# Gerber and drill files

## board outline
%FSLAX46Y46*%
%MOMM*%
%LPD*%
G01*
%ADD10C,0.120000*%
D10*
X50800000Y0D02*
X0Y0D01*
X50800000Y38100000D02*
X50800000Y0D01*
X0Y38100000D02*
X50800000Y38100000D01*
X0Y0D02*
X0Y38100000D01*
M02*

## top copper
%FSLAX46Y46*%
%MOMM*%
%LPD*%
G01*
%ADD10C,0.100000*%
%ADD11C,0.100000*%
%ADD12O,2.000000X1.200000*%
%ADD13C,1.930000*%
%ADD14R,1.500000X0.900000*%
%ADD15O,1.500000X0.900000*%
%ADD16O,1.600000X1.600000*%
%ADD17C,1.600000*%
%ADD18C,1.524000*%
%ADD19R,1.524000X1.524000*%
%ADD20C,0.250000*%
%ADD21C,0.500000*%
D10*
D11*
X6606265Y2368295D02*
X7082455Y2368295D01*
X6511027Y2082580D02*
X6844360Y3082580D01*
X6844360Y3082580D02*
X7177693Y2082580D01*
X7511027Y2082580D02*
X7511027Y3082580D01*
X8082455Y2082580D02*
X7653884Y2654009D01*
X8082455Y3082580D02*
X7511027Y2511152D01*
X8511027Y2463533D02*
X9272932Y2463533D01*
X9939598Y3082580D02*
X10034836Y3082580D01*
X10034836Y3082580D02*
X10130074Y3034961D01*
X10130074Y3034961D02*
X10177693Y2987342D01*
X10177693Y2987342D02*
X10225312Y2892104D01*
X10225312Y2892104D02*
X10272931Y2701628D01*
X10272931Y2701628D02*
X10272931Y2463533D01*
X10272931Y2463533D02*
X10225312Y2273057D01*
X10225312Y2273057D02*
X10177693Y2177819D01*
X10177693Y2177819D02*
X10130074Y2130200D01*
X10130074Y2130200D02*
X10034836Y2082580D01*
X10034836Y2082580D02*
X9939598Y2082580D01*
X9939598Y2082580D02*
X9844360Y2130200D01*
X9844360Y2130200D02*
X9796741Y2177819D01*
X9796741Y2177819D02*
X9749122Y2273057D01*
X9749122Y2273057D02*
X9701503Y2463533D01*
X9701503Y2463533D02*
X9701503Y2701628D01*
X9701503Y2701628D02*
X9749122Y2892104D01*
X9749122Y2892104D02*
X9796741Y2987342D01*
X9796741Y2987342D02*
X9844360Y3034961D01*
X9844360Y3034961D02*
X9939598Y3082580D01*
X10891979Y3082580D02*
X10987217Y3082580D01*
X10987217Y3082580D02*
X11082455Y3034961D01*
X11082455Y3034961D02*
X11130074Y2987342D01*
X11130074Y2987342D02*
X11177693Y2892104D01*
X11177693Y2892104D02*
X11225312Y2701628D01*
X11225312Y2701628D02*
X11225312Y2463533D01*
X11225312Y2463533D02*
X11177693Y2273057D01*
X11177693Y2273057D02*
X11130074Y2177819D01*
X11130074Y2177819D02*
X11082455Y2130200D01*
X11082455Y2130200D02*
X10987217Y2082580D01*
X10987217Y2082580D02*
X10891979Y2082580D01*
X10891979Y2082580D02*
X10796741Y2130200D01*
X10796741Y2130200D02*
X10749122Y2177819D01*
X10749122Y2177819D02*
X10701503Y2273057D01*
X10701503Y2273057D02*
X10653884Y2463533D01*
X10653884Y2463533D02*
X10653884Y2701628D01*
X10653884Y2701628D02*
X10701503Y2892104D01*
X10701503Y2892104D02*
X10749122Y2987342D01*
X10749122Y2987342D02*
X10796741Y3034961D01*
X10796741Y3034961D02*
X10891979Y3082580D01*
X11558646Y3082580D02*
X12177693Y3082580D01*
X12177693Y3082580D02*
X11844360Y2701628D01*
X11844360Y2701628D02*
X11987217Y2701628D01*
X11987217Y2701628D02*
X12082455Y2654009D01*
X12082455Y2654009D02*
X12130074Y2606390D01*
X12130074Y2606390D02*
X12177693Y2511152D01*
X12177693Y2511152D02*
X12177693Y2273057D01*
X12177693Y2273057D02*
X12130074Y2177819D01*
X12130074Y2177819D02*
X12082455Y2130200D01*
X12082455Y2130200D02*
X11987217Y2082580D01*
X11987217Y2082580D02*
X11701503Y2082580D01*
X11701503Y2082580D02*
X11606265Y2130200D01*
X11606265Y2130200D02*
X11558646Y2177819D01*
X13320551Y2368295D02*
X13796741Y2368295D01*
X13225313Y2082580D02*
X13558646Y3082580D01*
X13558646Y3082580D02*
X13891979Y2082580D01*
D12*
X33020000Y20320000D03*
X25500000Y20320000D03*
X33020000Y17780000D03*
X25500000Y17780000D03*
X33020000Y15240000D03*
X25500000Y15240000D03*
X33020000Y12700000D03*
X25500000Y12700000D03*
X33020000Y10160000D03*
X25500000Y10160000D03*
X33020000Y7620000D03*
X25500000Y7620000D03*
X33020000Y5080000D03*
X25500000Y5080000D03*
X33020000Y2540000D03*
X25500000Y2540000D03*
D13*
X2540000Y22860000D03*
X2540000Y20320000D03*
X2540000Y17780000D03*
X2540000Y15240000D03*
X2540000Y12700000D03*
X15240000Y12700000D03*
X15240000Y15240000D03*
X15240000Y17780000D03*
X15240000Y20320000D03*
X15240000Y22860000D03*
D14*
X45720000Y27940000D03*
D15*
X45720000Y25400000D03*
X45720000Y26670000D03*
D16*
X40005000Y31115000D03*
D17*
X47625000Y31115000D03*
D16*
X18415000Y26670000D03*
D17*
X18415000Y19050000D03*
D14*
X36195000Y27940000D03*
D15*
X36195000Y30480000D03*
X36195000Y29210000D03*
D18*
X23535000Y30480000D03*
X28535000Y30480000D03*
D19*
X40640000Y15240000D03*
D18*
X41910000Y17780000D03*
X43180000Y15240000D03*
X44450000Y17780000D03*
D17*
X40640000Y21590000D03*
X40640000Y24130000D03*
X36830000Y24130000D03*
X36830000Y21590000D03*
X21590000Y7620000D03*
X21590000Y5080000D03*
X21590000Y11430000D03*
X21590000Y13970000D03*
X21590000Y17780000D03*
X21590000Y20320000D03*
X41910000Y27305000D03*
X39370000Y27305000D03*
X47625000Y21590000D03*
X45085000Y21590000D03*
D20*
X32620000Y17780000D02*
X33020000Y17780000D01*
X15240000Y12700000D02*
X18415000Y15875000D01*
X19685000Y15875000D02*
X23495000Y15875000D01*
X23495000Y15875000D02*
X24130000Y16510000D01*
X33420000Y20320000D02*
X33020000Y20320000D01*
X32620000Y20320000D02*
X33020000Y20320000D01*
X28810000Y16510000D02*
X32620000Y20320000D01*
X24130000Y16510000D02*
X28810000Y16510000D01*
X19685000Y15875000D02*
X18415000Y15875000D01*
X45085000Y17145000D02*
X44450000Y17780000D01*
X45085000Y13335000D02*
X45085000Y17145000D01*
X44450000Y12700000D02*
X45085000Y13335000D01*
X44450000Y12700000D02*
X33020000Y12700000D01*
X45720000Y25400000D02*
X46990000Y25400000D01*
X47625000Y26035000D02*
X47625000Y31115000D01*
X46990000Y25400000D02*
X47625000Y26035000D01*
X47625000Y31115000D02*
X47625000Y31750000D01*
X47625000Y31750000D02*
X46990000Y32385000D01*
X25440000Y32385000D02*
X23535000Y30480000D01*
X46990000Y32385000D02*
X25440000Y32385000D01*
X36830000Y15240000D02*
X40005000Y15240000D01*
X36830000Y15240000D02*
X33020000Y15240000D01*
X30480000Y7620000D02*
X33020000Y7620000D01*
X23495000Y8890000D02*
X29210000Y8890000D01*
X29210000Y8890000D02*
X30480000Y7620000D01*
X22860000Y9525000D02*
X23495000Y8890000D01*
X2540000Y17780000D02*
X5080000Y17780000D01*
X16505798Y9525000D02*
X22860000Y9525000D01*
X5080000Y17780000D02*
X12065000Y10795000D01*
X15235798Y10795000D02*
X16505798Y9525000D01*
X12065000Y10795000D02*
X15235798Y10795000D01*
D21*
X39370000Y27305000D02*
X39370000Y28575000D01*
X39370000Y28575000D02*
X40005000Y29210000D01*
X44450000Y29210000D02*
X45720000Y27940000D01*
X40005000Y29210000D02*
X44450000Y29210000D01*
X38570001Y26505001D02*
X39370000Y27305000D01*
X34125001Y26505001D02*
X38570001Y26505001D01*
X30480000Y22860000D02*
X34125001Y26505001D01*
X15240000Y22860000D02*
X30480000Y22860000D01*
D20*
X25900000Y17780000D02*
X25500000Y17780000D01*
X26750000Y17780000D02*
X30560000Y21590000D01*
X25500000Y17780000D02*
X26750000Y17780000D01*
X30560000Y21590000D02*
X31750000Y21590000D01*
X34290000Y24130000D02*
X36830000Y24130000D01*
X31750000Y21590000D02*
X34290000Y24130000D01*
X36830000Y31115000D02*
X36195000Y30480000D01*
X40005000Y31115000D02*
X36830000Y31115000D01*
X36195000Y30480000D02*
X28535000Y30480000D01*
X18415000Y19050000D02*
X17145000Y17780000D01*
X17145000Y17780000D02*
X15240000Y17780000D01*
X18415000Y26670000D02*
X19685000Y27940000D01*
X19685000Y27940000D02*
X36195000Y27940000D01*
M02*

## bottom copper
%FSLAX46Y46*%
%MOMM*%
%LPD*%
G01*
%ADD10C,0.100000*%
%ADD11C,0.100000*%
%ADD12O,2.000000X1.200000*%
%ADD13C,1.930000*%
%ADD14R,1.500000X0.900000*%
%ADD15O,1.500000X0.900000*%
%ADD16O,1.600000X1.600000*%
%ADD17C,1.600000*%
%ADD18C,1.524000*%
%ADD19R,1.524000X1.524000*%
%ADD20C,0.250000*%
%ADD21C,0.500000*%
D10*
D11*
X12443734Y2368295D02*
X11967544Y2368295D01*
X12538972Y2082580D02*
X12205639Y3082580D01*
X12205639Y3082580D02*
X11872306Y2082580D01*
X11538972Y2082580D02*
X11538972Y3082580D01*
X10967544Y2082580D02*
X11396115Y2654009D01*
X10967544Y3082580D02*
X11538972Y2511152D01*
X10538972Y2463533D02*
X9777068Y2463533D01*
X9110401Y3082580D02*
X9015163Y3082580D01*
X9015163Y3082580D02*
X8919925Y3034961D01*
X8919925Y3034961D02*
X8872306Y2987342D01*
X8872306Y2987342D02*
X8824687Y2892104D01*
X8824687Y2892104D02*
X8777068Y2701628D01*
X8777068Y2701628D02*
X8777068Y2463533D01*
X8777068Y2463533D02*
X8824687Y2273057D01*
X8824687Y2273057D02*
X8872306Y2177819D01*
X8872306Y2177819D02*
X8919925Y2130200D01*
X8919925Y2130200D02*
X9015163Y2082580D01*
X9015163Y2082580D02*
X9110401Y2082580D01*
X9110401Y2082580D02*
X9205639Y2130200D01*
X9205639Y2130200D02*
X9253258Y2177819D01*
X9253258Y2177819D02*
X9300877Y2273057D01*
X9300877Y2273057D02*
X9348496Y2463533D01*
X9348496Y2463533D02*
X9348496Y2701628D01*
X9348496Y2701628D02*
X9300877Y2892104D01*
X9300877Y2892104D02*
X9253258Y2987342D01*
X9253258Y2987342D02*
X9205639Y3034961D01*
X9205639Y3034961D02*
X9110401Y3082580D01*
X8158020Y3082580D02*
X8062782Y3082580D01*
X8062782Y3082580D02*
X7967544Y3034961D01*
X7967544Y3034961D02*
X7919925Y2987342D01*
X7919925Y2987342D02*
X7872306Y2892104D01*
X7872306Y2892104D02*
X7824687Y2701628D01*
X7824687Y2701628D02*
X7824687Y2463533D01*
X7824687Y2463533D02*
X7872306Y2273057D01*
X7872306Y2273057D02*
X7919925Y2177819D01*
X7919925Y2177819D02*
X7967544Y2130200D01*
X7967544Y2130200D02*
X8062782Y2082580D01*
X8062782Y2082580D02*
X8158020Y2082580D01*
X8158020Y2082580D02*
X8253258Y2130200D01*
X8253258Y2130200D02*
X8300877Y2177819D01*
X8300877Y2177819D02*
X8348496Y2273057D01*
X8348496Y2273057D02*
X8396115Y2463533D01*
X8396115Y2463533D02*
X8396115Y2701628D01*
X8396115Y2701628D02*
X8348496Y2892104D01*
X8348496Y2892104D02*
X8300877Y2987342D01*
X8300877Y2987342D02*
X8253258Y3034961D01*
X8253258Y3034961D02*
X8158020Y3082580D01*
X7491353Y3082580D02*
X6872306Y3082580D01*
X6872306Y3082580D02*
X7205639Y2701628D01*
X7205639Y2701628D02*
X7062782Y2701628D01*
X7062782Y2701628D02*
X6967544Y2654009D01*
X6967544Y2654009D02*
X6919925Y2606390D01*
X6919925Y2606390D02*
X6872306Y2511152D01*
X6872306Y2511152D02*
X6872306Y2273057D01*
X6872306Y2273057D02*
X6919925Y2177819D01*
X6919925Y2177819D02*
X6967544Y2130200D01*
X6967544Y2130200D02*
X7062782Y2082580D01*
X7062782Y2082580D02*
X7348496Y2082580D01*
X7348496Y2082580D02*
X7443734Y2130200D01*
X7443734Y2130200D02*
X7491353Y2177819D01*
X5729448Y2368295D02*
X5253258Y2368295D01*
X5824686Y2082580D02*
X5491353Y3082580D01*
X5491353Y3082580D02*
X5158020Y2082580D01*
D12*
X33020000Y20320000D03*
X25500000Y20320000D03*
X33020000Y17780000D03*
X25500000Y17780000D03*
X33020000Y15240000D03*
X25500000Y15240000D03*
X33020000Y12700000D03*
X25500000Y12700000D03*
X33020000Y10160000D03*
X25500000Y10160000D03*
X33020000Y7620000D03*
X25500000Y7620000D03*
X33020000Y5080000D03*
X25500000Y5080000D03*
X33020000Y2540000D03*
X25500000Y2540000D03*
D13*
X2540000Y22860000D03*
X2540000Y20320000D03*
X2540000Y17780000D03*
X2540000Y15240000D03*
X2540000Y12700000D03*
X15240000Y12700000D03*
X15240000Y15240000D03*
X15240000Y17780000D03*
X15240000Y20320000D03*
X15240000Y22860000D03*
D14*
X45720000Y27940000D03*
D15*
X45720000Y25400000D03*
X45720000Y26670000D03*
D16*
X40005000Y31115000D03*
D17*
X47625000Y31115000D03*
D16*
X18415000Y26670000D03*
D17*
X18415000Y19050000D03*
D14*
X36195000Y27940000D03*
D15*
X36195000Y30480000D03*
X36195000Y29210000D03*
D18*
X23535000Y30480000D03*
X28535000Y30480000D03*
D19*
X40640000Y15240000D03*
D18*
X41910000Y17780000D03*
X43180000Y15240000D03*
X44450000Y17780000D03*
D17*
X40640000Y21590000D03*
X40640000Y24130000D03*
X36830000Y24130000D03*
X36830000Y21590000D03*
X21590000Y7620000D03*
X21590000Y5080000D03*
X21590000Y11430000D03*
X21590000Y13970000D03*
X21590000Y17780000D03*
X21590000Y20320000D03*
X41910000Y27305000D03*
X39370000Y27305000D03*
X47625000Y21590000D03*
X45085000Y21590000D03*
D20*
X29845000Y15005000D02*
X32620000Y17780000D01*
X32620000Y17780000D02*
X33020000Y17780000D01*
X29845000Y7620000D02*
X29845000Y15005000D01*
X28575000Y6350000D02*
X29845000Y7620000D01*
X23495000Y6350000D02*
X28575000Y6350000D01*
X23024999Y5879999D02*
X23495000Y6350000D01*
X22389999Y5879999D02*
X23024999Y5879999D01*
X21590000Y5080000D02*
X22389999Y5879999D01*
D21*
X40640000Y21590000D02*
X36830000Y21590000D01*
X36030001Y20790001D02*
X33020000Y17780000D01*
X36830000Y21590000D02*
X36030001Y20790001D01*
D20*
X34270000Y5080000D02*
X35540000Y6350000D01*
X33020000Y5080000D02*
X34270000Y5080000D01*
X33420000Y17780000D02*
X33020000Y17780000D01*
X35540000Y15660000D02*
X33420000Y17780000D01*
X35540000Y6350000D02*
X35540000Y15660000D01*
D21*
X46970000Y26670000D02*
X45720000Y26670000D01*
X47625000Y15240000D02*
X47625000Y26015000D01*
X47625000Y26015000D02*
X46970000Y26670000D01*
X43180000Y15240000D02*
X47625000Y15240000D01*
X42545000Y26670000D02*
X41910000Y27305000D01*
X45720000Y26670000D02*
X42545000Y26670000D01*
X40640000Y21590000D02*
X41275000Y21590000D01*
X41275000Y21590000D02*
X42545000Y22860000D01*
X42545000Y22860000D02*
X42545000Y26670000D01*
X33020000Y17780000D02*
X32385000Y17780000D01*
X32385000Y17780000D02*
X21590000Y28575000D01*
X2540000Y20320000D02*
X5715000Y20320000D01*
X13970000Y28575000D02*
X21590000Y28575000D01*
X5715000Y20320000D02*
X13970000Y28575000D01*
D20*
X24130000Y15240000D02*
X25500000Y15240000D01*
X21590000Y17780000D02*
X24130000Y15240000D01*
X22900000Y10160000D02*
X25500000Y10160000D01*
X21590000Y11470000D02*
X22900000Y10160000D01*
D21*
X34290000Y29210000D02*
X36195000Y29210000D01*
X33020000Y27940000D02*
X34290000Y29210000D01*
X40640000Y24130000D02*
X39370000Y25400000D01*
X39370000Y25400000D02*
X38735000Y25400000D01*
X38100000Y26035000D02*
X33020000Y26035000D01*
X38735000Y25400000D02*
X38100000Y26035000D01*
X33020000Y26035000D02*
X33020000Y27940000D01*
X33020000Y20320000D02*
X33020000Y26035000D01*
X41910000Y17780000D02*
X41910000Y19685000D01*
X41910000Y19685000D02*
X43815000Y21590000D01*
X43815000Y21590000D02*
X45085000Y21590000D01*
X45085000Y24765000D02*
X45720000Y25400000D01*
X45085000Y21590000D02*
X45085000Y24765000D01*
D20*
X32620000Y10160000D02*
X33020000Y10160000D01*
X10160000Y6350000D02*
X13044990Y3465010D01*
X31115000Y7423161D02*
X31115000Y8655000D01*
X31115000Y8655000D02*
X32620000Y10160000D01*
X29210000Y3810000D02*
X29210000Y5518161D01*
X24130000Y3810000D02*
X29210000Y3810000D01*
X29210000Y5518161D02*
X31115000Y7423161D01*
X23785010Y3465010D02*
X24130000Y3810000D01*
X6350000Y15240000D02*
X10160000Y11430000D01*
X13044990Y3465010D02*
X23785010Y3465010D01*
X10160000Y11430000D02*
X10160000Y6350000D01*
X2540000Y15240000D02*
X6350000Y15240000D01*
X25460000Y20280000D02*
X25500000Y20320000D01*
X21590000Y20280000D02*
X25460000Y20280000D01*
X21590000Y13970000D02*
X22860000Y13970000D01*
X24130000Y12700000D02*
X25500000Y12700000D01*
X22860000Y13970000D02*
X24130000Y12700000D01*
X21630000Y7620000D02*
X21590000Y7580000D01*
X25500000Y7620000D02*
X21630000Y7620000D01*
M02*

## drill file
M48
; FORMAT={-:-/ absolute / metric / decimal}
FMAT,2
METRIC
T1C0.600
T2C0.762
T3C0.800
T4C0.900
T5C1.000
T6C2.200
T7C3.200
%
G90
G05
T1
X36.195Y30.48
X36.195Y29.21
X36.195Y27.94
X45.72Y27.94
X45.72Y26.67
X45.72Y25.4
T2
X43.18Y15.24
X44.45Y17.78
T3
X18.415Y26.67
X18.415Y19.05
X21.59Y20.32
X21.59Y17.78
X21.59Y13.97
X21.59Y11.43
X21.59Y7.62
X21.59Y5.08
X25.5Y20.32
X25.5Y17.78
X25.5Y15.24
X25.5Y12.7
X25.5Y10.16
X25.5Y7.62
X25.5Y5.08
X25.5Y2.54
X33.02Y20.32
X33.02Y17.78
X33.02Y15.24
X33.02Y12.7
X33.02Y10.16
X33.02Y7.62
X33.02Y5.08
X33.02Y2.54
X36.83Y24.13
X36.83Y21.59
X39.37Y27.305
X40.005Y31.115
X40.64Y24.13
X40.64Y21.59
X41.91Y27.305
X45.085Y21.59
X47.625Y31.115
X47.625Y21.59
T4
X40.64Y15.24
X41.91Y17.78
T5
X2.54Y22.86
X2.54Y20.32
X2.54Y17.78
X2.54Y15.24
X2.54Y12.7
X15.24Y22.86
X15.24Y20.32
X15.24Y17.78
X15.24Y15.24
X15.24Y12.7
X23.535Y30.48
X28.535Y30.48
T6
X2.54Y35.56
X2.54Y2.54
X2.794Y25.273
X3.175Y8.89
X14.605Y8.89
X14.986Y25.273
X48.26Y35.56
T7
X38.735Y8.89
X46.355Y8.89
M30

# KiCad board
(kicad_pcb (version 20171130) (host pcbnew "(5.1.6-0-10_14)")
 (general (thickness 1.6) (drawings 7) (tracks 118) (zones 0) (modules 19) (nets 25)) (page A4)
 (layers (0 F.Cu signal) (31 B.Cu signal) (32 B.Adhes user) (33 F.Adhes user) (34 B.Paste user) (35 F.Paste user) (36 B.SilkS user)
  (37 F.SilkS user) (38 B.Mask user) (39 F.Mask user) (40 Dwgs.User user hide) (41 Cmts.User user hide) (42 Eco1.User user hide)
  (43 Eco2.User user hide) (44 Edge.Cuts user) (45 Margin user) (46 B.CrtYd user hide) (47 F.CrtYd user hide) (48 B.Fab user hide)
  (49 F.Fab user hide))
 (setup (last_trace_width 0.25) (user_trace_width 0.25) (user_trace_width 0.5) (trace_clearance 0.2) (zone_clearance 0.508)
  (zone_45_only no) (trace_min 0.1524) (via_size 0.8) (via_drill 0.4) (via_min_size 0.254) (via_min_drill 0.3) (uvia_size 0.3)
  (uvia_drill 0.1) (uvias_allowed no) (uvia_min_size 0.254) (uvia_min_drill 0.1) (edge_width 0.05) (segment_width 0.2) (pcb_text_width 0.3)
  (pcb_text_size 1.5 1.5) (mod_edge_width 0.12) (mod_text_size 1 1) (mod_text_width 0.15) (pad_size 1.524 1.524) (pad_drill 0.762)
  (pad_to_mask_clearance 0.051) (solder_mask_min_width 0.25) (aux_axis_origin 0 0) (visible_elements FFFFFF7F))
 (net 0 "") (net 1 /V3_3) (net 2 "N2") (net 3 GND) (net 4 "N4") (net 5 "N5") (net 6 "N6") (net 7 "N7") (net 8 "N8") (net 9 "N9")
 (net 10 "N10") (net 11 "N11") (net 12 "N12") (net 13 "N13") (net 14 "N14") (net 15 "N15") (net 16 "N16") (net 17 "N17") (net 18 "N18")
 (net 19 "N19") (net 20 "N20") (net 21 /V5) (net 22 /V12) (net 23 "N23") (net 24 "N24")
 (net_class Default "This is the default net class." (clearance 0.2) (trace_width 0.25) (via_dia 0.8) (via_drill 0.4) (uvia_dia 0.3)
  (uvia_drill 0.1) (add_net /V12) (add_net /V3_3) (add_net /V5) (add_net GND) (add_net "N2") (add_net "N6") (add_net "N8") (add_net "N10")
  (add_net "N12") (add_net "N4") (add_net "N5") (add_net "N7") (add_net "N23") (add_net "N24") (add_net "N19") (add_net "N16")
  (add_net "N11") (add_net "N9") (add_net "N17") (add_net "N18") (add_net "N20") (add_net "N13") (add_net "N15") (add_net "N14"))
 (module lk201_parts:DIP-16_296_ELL (layer F.Cu) (at 29.26 -11.43 270)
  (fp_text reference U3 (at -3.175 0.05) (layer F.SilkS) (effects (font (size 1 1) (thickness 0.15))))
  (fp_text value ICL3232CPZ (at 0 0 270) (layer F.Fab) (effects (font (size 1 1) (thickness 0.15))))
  (pad 16 thru_hole oval (at -8.89 -3.76 270) (size 1.2 2) (drill 0.8) (layers *.Cu *.Mask) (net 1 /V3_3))
  (pad 1 thru_hole oval (at -8.89 3.76 270) (size 1.2 2) (drill 0.8) (layers *.Cu *.Mask) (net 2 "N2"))
  (pad 15 thru_hole oval (at -6.35 -3.76 270) (size 1.2 2) (drill 0.8) (layers *.Cu *.Mask) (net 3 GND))
  (pad 2 thru_hole oval (at -6.35 3.76 270) (size 1.2 2) (drill 0.8) (layers *.Cu *.Mask) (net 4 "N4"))
  (pad 14 thru_hole oval (at -3.81 -3.76 270) (size 1.2 2) (drill 0.8) (layers *.Cu *.Mask) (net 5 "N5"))
  (pad 3 thru_hole oval (at -3.81 3.76 270) (size 1.2 2) (drill 0.8) (layers *.Cu *.Mask) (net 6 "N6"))
  (pad 13 thru_hole oval (at -1.27 -3.76 270) (size 1.2 2) (drill 0.8) (layers *.Cu *.Mask) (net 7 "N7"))
  (pad 4 thru_hole oval (at -1.27 3.76 270) (size 1.2 2) (drill 0.8) (layers *.Cu *.Mask) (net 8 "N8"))
  (pad 12 thru_hole oval (at 1.27 -3.76 270) (size 1.2 2) (drill 0.8) (layers *.Cu *.Mask) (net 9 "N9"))
  (pad 5 thru_hole oval (at 1.27 3.76 270) (size 1.2 2) (drill 0.8) (layers *.Cu *.Mask) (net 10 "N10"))
  (pad 11 thru_hole oval (at 3.81 -3.76 270) (size 1.2 2) (drill 0.8) (layers *.Cu *.Mask) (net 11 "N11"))
  (pad 6 thru_hole oval (at 3.81 3.76 270) (size 1.2 2) (drill 0.8) (layers *.Cu *.Mask) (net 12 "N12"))
  (pad 10 thru_hole oval (at 6.35 -3.76 270) (size 1.2 2) (drill 0.8) (layers *.Cu *.Mask) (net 3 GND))
  (pad 7 thru_hole oval (at 6.35 3.76 270) (size 1.2 2) (drill 0.8) (layers *.Cu *.Mask) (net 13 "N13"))
  (pad 9 thru_hole oval (at 8.89 -3.76 270) (size 1.2 2) (drill 0.8) (layers *.Cu *.Mask) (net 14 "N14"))
  (pad 8 thru_hole oval (at 8.89 3.76 270) (size 1.2 2) (drill 0.8) (layers *.Cu *.Mask) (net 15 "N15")))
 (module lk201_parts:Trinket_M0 (layer F.Cu) (at 8.89 -19.05 180)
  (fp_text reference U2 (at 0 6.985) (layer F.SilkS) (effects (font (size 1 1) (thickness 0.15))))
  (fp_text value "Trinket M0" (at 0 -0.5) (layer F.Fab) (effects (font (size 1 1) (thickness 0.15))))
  (pad "" np_thru_hole circle (at -6.096 6.223 180) (size 2.2 2.2) (drill 2.2) (layers *.Mask F.Cu))
  (pad "" np_thru_hole circle (at 6.096 6.223 180) (size 2.2 2.2) (drill 2.2) (layers *.Mask F.Cu))
  (pad "" np_thru_hole circle (at 5.715 -10.16 180) (size 2.2 2.2) (drill 2.2) (layers *.Mask F.Cu))
  (pad "" np_thru_hole circle (at -5.715 -10.16 180) (size 2.2 2.2) (drill 2.2) (layers *.Mask F.Cu))
  (pad 1 thru_hole circle (at 6.35 3.81 180) (size 1.93 1.93) (drill 1) (layers *.Cu *.Mask) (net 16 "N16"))
  (pad 2 thru_hole circle (at 6.35 1.27 180) (size 1.93 1.93) (drill 1) (layers *.Cu *.Mask) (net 3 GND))
  (pad 3 thru_hole circle (at 6.35 -1.27 180) (size 1.93 1.93) (drill 1) (layers *.Cu *.Mask) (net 11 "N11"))
  (pad 4 thru_hole circle (at 6.35 -3.81 180) (size 1.93 1.93) (drill 1) (layers *.Cu *.Mask) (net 9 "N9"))
  (pad 5 thru_hole circle (at 6.35 -6.35 180) (size 1.93 1.93) (drill 1) (layers *.Cu *.Mask) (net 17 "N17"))
  (pad 6 thru_hole circle (at -6.35 -6.35 180) (size 1.93 1.93) (drill 1) (layers *.Cu *.Mask) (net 1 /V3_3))
  (pad 7 thru_hole circle (at -6.35 -3.81 180) (size 1.93 1.93) (drill 1) (layers *.Cu *.Mask) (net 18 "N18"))
  (pad 8 thru_hole circle (at -6.35 -1.27 180) (size 1.93 1.93) (drill 1) (layers *.Cu *.Mask) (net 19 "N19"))
  (pad 9 thru_hole circle (at -6.35 1.27 180) (size 1.93 1.93) (drill 1) (layers *.Cu *.Mask) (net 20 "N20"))
  (pad 10 thru_hole circle (at -6.35 3.81 180) (size 1.93 1.93) (drill 1) (layers *.Cu *.Mask) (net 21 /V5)))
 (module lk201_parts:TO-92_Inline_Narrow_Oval (layer F.Cu) (at 45.72 -27.94 270)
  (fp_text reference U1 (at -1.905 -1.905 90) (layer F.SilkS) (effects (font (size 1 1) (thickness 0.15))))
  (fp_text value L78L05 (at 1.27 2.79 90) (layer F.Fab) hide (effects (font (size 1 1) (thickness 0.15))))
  (pad 1 thru_hole rect (at 0 0 90) (size 0.9 1.5) (drill 0.6) (layers *.Cu *.Mask) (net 21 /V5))
  (pad 3 thru_hole oval (at 2.54 0 90) (size 0.9 1.5) (drill 0.6) (layers *.Cu *.Mask) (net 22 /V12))
  (pad 2 thru_hole oval (at 1.27 0 90) (size 0.9 1.5) (drill 0.6) (layers *.Cu *.Mask) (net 3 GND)))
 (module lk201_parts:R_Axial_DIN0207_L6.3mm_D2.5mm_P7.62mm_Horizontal (layer F.Cu) (at 47.625 -31.115 180)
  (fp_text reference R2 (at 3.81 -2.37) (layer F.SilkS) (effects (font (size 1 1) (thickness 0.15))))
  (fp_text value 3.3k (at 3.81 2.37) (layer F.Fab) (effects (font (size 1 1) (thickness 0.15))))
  (pad 2 thru_hole oval (at 7.62 0 180) (size 1.6 1.6) (drill 0.8) (layers *.Cu *.Mask) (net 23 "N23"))
  (pad 1 thru_hole circle (at 0 0 180) (size 1.6 1.6) (drill 0.8) (layers *.Cu *.Mask) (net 22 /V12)))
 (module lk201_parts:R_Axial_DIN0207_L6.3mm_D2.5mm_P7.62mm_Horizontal (layer F.Cu) (at 18.415 -19.05 90)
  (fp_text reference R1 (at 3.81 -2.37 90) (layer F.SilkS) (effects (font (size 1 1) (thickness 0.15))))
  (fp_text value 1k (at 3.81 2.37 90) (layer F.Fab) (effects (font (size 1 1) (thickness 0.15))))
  (pad 2 thru_hole oval (at 7.62 0 90) (size 1.6 1.6) (drill 0.8) (layers *.Cu *.Mask) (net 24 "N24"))
  (pad 1 thru_hole circle (at 0 0 90) (size 1.6 1.6) (drill 0.8) (layers *.Cu *.Mask) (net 19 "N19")))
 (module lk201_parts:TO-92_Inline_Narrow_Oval (layer F.Cu) (at 36.195 -27.94 90)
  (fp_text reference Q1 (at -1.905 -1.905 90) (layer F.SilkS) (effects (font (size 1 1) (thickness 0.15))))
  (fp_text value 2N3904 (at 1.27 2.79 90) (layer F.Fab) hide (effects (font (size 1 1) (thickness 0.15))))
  (pad 1 thru_hole rect (at 0 0 270) (size 0.9 1.5) (drill 0.6) (layers *.Cu *.Mask) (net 24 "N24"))
  (pad 3 thru_hole oval (at 2.54 0 270) (size 0.9 1.5) (drill 0.6) (layers *.Cu *.Mask) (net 23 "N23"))
  (pad 2 thru_hole oval (at 1.27 0 270) (size 0.9 1.5) (drill 0.6) (layers *.Cu *.Mask) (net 1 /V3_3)))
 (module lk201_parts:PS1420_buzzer (layer F.Cu) (at 26.035 -30.48 180)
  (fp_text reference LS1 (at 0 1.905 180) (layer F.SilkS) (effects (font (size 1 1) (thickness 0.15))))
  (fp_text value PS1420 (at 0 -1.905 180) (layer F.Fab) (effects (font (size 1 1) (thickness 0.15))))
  (pad 1 thru_hole circle (at 2.5 0 180) (size 1.524 1.524) (drill 1) (layers *.Cu *.Mask) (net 22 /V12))
  (pad 2 thru_hole circle (at -2.5 0 180) (size 1.524 1.524) (drill 1) (layers *.Cu *.Mask) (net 23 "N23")))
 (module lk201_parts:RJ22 (layer F.Cu) (at 42.545 -8.89)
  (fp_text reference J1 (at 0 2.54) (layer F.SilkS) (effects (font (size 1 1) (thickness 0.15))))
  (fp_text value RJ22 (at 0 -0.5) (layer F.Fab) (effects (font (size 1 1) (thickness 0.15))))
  (pad 1 thru_hole rect (at -1.905 -6.35) (size 1.524 1.524) (drill 0.9) (layers *.Cu *.Mask) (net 5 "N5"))
  (pad 2 thru_hole circle (at -0.635 -8.89) (size 1.524 1.524) (drill 0.9) (layers *.Cu *.Mask) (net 22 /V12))
  (pad 3 thru_hole circle (at 0.635 -6.35) (size 1.524 1.524) (drill 0.762) (layers *.Cu *.Mask) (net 3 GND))
  (pad 4 thru_hole circle (at 1.905 -8.89) (size 1.524 1.524) (drill 0.762) (layers *.Cu *.Mask) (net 7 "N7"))
  (pad "" np_thru_hole circle (at 3.81 0) (size 3.2 3.2) (drill 3.2) (layers *.Mask F.Cu))
  (pad "" np_thru_hole circle (at -3.81 0) (size 3.2 3.2) (drill 3.2) (layers *.Mask F.Cu)))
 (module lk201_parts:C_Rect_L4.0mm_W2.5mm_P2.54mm (layer F.Cu) (at 40.64 -24.13 270)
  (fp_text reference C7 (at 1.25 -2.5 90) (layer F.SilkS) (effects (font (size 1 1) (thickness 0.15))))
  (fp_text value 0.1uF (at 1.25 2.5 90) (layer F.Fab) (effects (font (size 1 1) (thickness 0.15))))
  (pad 2 thru_hole circle (at 2.54 0 270) (size 1.6 1.6) (drill 0.8) (layers *.Cu *.Mask) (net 3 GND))
  (pad 1 thru_hole circle (at 0 0 270) (size 1.6 1.6) (drill 0.8) (layers *.Cu *.Mask) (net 1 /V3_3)))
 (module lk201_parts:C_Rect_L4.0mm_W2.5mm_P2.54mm (layer F.Cu) (at 36.83 -21.59 90)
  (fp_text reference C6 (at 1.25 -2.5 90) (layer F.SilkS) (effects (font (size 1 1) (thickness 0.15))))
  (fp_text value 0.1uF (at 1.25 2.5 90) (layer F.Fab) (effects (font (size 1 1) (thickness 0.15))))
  (pad 2 thru_hole circle (at 2.54 0 90) (size 1.6 1.6) (drill 0.8) (layers *.Cu *.Mask) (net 4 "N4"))
  (pad 1 thru_hole circle (at 0 0 90) (size 1.6 1.6) (drill 0.8) (layers *.Cu *.Mask) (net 3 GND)))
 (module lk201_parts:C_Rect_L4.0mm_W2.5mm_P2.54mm (layer F.Cu) (at 21.59 -5.08 90)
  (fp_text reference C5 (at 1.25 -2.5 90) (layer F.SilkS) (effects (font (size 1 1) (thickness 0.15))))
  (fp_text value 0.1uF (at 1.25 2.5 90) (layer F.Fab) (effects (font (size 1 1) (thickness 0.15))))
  (pad 2 thru_hole circle (at 2.54 0 90) (size 1.6 1.6) (drill 0.8) (layers *.Cu *.Mask) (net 12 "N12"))
  (pad 1 thru_hole circle (at 0 0 90) (size 1.6 1.6) (drill 0.8) (layers *.Cu *.Mask) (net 3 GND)))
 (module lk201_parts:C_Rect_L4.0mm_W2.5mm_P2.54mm (layer F.Cu) (at 21.59 -13.97 270)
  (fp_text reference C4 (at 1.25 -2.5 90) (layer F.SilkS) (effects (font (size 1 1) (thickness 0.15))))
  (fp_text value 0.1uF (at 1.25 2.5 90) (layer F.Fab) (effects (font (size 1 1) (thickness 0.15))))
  (pad 2 thru_hole circle (at 2.54 0 270) (size 1.6 1.6) (drill 0.8) (layers *.Cu *.Mask) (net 10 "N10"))
  (pad 1 thru_hole circle (at 0 0 270) (size 1.6 1.6) (drill 0.8) (layers *.Cu *.Mask) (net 8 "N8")))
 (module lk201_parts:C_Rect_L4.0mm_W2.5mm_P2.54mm (layer F.Cu) (at 21.59 -20.32 270)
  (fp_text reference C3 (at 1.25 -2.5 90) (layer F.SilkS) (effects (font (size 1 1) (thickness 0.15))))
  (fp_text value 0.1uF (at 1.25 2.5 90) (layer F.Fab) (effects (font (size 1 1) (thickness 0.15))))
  (pad 2 thru_hole circle (at 2.54 0 270) (size 1.6 1.6) (drill 0.8) (layers *.Cu *.Mask) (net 6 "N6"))
  (pad 1 thru_hole circle (at 0 0 270) (size 1.6 1.6) (drill 0.8) (layers *.Cu *.Mask) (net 2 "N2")))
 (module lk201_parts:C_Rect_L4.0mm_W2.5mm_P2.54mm (layer F.Cu) (at 39.37 -27.305)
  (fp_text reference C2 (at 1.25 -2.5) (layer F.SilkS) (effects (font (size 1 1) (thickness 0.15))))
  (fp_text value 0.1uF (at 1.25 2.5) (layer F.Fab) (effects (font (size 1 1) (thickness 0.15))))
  (pad 2 thru_hole circle (at 2.54 0) (size 1.6 1.6) (drill 0.8) (layers *.Cu *.Mask) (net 3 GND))
  (pad 1 thru_hole circle (at 0 0) (size 1.6 1.6) (drill 0.8) (layers *.Cu *.Mask) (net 21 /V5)))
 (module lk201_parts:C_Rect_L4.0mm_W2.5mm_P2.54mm (layer F.Cu) (at 45.085 -21.59)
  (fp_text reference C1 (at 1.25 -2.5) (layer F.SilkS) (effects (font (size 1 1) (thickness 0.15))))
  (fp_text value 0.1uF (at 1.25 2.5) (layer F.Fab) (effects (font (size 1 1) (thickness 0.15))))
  (pad 2 thru_hole circle (at 2.54 0) (size 1.6 1.6) (drill 0.8) (layers *.Cu *.Mask) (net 3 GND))
  (pad 1 thru_hole circle (at 0 0) (size 1.6 1.6) (drill 0.8) (layers *.Cu *.Mask) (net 22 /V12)))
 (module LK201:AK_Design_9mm (layer F.Cu) (at 33.655 -33.655)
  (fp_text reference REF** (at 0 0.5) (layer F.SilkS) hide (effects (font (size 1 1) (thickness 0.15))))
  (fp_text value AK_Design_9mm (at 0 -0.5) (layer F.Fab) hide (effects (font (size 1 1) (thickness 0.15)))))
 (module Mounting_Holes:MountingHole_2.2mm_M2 (layer F.Cu) (at 2.54 -2.54)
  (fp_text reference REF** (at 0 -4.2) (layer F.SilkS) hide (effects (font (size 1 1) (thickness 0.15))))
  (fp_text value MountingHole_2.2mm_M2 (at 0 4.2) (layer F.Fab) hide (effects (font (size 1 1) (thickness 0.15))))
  (pad 1 np_thru_hole circle (at 0 0) (size 2.2 2.2) (drill 2.2) (layers *.Cu *.Mask)))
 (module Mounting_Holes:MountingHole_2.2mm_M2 (layer F.Cu) (at 2.54 -35.56)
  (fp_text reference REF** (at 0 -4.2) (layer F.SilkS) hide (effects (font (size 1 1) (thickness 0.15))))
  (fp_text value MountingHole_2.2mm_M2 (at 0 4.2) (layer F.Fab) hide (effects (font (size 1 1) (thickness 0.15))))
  (pad 1 np_thru_hole circle (at 0 0) (size 2.2 2.2) (drill 2.2) (layers *.Cu *.Mask)))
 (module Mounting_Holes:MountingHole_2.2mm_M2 (layer F.Cu) (at 48.26 -35.56)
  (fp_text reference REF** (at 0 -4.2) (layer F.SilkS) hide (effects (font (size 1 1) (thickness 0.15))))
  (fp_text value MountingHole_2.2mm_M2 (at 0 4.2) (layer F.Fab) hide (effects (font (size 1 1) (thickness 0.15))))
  (pad 1 np_thru_hole circle (at 0 0) (size 2.2 2.2) (drill 2.2) (layers *.Cu *.Mask)))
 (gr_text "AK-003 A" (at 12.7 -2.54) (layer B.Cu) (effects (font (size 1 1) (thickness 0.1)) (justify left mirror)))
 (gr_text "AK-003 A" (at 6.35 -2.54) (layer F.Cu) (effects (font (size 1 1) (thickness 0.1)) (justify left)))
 (gr_line (start 50.8 0) (end 0 0) (layer Edge.Cuts) (width 0.12))
 (gr_line (start 50.8 -38.1) (end 50.8 0) (layer Edge.Cuts) (width 0.12))
 (gr_line (start 0 -38.1) (end 50.8 -38.1) (layer Edge.Cuts) (width 0.12))
 (gr_line (start 0 0) (end 0 -38.1) (layer Edge.Cuts) (width 0.12))
 (segment (start 29.845 -15.005) (end 32.62 -17.78) (width 0.25) (layer B.Cu) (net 3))
 (segment (start 32.62 -17.78) (end 33.02 -17.78) (width 0.25) (layer B.Cu) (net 3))
 (segment (start 29.845 -7.62) (end 29.845 -15.005) (width 0.25) (layer B.Cu) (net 3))
 (segment (start 28.575 -6.35) (end 29.845 -7.62) (width 0.25) (layer B.Cu) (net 3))
 (segment (start 23.495 -6.35) (end 28.575 -6.35) (width 0.25) (layer B.Cu) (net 3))
 (segment (start 23.024999 -5.879999) (end 23.495 -6.35) (width 0.25) (layer B.Cu) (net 3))
 (segment (start 22.389999 -5.879999) (end 23.024999 -5.879999) (width 0.25) (layer B.Cu) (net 3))
 (segment (start 21.59 -5.08) (end 22.389999 -5.879999) (width 0.25) (layer B.Cu) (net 3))
 (segment (start 32.62 -17.78) (end 33.02 -17.78) (width 0.25) (layer F.Cu) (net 3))
 (segment (start 40.64 -21.59) (end 36.83 -21.59) (width 0.5) (layer B.Cu) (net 3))
 (segment (start 36.030001 -20.790001) (end 33.02 -17.78) (width 0.5) (layer B.Cu) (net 3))
 (segment (start 36.83 -21.59) (end 36.030001 -20.790001) (width 0.5) (layer B.Cu) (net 3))
 (segment (start 34.27 -5.08) (end 35.54 -6.35) (width 0.25) (layer B.Cu) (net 3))
 (segment (start 33.02 -5.08) (end 34.27 -5.08) (width 0.25) (layer B.Cu) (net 3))
 (segment (start 33.42 -17.78) (end 33.02 -17.78) (width 0.25) (layer B.Cu) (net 3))
 (segment (start 35.54 -15.66) (end 33.42 -17.78) (width 0.25) (layer B.Cu) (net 3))
 (segment (start 35.54 -6.35) (end 35.54 -15.66) (width 0.25) (layer B.Cu) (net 3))
 (segment (start 46.97 -26.67) (end 45.72 -26.67) (width 0.5) (layer B.Cu) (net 3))
 (segment (start 47.625 -15.24) (end 47.625 -26.015) (width 0.5) (layer B.Cu) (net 3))
 (segment (start 47.625 -26.015) (end 46.97 -26.67) (width 0.5) (layer B.Cu) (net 3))
 (segment (start 43.18 -15.24) (end 47.625 -15.24) (width 0.5) (layer B.Cu) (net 3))
 (segment (start 42.545 -26.67) (end 41.91 -27.305) (width 0.5) (layer B.Cu) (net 3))
 (segment (start 45.72 -26.67) (end 42.545 -26.67) (width 0.5) (layer B.Cu) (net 3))
 (segment (start 40.64 -21.59) (end 41.275 -21.59) (width 0.5) (layer B.Cu) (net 3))
 (segment (start 41.275 -21.59) (end 42.545 -22.86) (width 0.5) (layer B.Cu) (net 3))
 (segment (start 42.545 -22.86) (end 42.545 -26.67) (width 0.5) (layer B.Cu) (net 3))
 (segment (start 33.02 -17.78) (end 32.385 -17.78) (width 0.5) (layer B.Cu) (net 3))
 (segment (start 32.385 -17.78) (end 21.59 -28.575) (width 0.5) (layer B.Cu) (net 3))
 (segment (start 2.54 -20.32) (end 5.715 -20.32) (width 0.5) (layer B.Cu) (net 3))
 (segment (start 13.97 -28.575) (end 21.59 -28.575) (width 0.5) (layer B.Cu) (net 3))
 (segment (start 5.715 -20.32) (end 13.97 -28.575) (width 0.5) (layer B.Cu) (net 3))
 (segment (start 24.13 -15.24) (end 25.5 -15.24) (width 0.25) (layer B.Cu) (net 6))
 (segment (start 21.59 -17.78) (end 24.13 -15.24) (width 0.25) (layer B.Cu) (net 6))
 (segment (start 22.9 -10.16) (end 25.5 -10.16) (width 0.25) (layer B.Cu) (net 10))
 (segment (start 21.59 -11.47) (end 22.9 -10.16) (width 0.25) (layer B.Cu) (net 10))
 (segment (start 15.24 -12.7) (end 18.415 -15.875) (width 0.25) (layer F.Cu) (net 1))
 (segment (start 19.685 -15.875) (end 23.495 -15.875) (width 0.25) (layer F.Cu) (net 1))
 (segment (start 23.495 -15.875) (end 24.13 -16.51) (width 0.25) (layer F.Cu) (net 1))
 (segment (start 33.42 -20.32) (end 33.02 -20.32) (width 0.25) (layer F.Cu) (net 1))
 (segment (start 32.62 -20.32) (end 33.02 -20.32) (width 0.25) (layer F.Cu) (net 1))
 (segment (start 28.81 -16.51) (end 32.62 -20.32) (width 0.25) (layer F.Cu) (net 1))
 (segment (start 24.13 -16.51) (end 28.81 -16.51) (width 0.25) (layer F.Cu) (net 1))
 (segment (start 34.29 -29.21) (end 36.195 -29.21) (width 0.5) (layer B.Cu) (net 1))
 (segment (start 33.02 -27.94) (end 34.29 -29.21) (width 0.5) (layer B.Cu) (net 1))
 (segment (start 40.64 -24.13) (end 39.37 -25.4) (width 0.5) (layer B.Cu) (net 1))
 (segment (start 39.37 -25.4) (end 38.735 -25.4) (width 0.5) (layer B.Cu) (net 1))
 (segment (start 38.1 -26.035) (end 33.02 -26.035) (width 0.5) (layer B.Cu) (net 1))
 (segment (start 38.735 -25.4) (end 38.1 -26.035) (width 0.5) (layer B.Cu) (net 1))
 (segment (start 33.02 -26.035) (end 33.02 -27.94) (width 0.5) (layer B.Cu) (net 1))
 (segment (start 33.02 -20.32) (end 33.02 -26.035) (width 0.5) (layer B.Cu) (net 1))
 (segment (start 19.685 -15.875) (end 18.415 -15.875) (width 0.25) (layer F.Cu) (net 1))
 (segment (start 45.085 -17.145) (end 44.45 -17.78) (width 0.25) (layer F.Cu) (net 7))
 (segment (start 45.085 -13.335) (end 45.085 -17.145) (width 0.25) (layer F.Cu) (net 7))
 (segment (start 44.45 -12.7) (end 45.085 -13.335) (width 0.25) (layer F.Cu) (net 7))
 (segment (start 44.45 -12.7) (end 33.02 -12.7) (width 0.25) (layer F.Cu) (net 7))
 (segment (start 41.91 -17.78) (end 41.91 -19.685) (width 0.5) (layer B.Cu) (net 22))
 (segment (start 41.91 -19.685) (end 43.815 -21.59) (width 0.5) (layer B.Cu) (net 22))
 (segment (start 43.815 -21.59) (end 45.085 -21.59) (width 0.5) (layer B.Cu) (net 22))
 (segment (start 45.085 -24.765) (end 45.72 -25.4) (width 0.5) (layer B.Cu) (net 22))
 (segment (start 45.085 -21.59) (end 45.085 -24.765) (width 0.5) (layer B.Cu) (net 22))
 (segment (start 45.72 -25.4) (end 46.99 -25.4) (width 0.25) (layer F.Cu) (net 22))
 (segment (start 47.625 -26.035) (end 47.625 -31.115) (width 0.25) (layer F.Cu) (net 22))
 (segment (start 46.99 -25.4) (end 47.625 -26.035) (width 0.25) (layer F.Cu) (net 22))
 (segment (start 47.625 -31.115) (end 47.625 -31.75) (width 0.25) (layer F.Cu) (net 22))
 (segment (start 47.625 -31.75) (end 46.99 -32.385) (width 0.25) (layer F.Cu) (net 22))
 (segment (start 25.44 -32.385) (end 23.535 -30.48) (width 0.25) (layer F.Cu) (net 22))
 (segment (start 46.99 -32.385) (end 25.44 -32.385) (width 0.25) (layer F.Cu) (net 22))
 (segment (start 36.83 -15.24) (end 40.005 -15.24) (width 0.25) (layer F.Cu) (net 5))
 (segment (start 36.83 -15.24) (end 33.02 -15.24) (width 0.25) (layer F.Cu) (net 5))
 (segment (start 32.62 -10.16) (end 33.02 -10.16) (width 0.25) (layer B.Cu) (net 9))
 (segment (start 10.16 -6.35) (end 13.04499 -3.46501) (width 0.25) (layer B.Cu) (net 9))
 (segment (start 31.115 -7.423161) (end 31.115 -8.655) (width 0.25) (layer B.Cu) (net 9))
 (segment (start 31.115 -8.655) (end 32.62 -10.16) (width 0.25) (layer B.Cu) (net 9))
 (segment (start 29.21 -3.81) (end 29.21 -5.518161) (width 0.25) (layer B.Cu) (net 9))
 (segment (start 24.13 -3.81) (end 29.21 -3.81) (width 0.25) (layer B.Cu) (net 9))
 (segment (start 29.21 -5.518161) (end 31.115 -7.423161) (width 0.25) (layer B.Cu) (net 9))
 (segment (start 23.78501 -3.46501) (end 24.13 -3.81) (width 0.25) (layer B.Cu) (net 9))
 (segment (start 6.35 -15.24) (end 10.16 -11.43) (width 0.25) (layer B.Cu) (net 9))
 (segment (start 13.04499 -3.46501) (end 23.78501 -3.46501) (width 0.25) (layer B.Cu) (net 9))
 (segment (start 10.16 -11.43) (end 10.16 -6.35) (width 0.25) (layer B.Cu) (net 9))
 (segment (start 2.54 -15.24) (end 6.35 -15.24) (width 0.25) (layer B.Cu) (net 9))
 (segment (start 30.48 -7.62) (end 33.02 -7.62) (width 0.25) (layer F.Cu) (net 11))
 (segment (start 23.495 -8.89) (end 29.21 -8.89) (width 0.25) (layer F.Cu) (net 11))
 (segment (start 29.21 -8.89) (end 30.48 -7.62) (width 0.25) (layer F.Cu) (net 11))
 (segment (start 22.86 -9.525) (end 23.495 -8.89) (width 0.25) (layer F.Cu) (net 11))
 (segment (start 2.54 -17.78) (end 5.08 -17.78) (width 0.25) (layer F.Cu) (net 11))
 (segment (start 16.505798 -9.525) (end 22.86 -9.525) (width 0.25) (layer F.Cu) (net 11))
 (segment (start 5.08 -17.78) (end 12.065 -10.795) (width 0.25) (layer F.Cu) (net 11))
 (segment (start 15.235798 -10.795) (end 16.505798 -9.525) (width 0.25) (layer F.Cu) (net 11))
 (segment (start 12.065 -10.795) (end 15.235798 -10.795) (width 0.25) (layer F.Cu) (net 11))
 (segment (start 39.37 -27.305) (end 39.37 -28.575) (width 0.5) (layer F.Cu) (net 21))
 (segment (start 39.37 -28.575) (end 40.005 -29.21) (width 0.5) (layer F.Cu) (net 21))
 (segment (start 44.45 -29.21) (end 45.72 -27.94) (width 0.5) (layer F.Cu) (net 21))
 (segment (start 40.005 -29.21) (end 44.45 -29.21) (width 0.5) (layer F.Cu) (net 21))
 (segment (start 38.570001 -26.505001) (end 39.37 -27.305) (width 0.5) (layer F.Cu) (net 21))
 (segment (start 34.125001 -26.505001) (end 38.570001 -26.505001) (width 0.5) (layer F.Cu) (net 21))
 (segment (start 30.48 -22.86) (end 34.125001 -26.505001) (width 0.5) (layer F.Cu) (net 21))
 (segment (start 15.24 -22.86) (end 30.48 -22.86) (width 0.5) (layer F.Cu) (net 21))
 (segment (start 25.46 -20.28) (end 25.5 -20.32) (width 0.25) (layer B.Cu) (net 2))
 (segment (start 21.59 -20.28) (end 25.46 -20.28) (width 0.25) (layer B.Cu) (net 2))
 (segment (start 21.59 -13.97) (end 22.86 -13.97) (width 0.25) (layer B.Cu) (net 8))
 (segment (start 24.13 -12.7) (end 25.5 -12.7) (width 0.25) (layer B.Cu) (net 8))
 (segment (start 22.86 -13.97) (end 24.13 -12.7) (width 0.25) (layer B.Cu) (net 8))
 (segment (start 21.63 -7.62) (end 21.59 -7.58) (width 0.25) (layer B.Cu) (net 12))
 (segment (start 25.5 -7.62) (end 21.63 -7.62) (width 0.25) (layer B.Cu) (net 12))
 (segment (start 25.9 -17.78) (end 25.5 -17.78) (width 0.25) (layer F.Cu) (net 4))
 (segment (start 26.75 -17.78) (end 30.56 -21.59) (width 0.25) (layer F.Cu) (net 4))
 (segment (start 25.5 -17.78) (end 26.75 -17.78) (width 0.25) (layer F.Cu) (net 4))
 (segment (start 30.56 -21.59) (end 31.75 -21.59) (width 0.25) (layer F.Cu) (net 4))
 (segment (start 34.29 -24.13) (end 36.83 -24.13) (width 0.25) (layer F.Cu) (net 4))
 (segment (start 31.75 -21.59) (end 34.29 -24.13) (width 0.25) (layer F.Cu) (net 4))
 (segment (start 36.83 -31.115) (end 36.195 -30.48) (width 0.25) (layer F.Cu) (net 23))
 (segment (start 40.005 -31.115) (end 36.83 -31.115) (width 0.25) (layer F.Cu) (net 23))
 (segment (start 36.195 -30.48) (end 28.535 -30.48) (width 0.25) (layer F.Cu) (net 23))
 (segment (start 18.415 -19.05) (end 17.145 -17.78) (width 0.25) (layer F.Cu) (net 19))
 (segment (start 17.145 -17.78) (end 15.24 -17.78) (width 0.25) (layer F.Cu) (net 19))
 (segment (start 18.415 -26.67) (end 19.685 -27.94) (width 0.25) (layer F.Cu) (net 24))
 (segment (start 19.685 -27.94) (end 36.195 -27.94) (width 0.25) (layer F.Cu) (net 24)))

